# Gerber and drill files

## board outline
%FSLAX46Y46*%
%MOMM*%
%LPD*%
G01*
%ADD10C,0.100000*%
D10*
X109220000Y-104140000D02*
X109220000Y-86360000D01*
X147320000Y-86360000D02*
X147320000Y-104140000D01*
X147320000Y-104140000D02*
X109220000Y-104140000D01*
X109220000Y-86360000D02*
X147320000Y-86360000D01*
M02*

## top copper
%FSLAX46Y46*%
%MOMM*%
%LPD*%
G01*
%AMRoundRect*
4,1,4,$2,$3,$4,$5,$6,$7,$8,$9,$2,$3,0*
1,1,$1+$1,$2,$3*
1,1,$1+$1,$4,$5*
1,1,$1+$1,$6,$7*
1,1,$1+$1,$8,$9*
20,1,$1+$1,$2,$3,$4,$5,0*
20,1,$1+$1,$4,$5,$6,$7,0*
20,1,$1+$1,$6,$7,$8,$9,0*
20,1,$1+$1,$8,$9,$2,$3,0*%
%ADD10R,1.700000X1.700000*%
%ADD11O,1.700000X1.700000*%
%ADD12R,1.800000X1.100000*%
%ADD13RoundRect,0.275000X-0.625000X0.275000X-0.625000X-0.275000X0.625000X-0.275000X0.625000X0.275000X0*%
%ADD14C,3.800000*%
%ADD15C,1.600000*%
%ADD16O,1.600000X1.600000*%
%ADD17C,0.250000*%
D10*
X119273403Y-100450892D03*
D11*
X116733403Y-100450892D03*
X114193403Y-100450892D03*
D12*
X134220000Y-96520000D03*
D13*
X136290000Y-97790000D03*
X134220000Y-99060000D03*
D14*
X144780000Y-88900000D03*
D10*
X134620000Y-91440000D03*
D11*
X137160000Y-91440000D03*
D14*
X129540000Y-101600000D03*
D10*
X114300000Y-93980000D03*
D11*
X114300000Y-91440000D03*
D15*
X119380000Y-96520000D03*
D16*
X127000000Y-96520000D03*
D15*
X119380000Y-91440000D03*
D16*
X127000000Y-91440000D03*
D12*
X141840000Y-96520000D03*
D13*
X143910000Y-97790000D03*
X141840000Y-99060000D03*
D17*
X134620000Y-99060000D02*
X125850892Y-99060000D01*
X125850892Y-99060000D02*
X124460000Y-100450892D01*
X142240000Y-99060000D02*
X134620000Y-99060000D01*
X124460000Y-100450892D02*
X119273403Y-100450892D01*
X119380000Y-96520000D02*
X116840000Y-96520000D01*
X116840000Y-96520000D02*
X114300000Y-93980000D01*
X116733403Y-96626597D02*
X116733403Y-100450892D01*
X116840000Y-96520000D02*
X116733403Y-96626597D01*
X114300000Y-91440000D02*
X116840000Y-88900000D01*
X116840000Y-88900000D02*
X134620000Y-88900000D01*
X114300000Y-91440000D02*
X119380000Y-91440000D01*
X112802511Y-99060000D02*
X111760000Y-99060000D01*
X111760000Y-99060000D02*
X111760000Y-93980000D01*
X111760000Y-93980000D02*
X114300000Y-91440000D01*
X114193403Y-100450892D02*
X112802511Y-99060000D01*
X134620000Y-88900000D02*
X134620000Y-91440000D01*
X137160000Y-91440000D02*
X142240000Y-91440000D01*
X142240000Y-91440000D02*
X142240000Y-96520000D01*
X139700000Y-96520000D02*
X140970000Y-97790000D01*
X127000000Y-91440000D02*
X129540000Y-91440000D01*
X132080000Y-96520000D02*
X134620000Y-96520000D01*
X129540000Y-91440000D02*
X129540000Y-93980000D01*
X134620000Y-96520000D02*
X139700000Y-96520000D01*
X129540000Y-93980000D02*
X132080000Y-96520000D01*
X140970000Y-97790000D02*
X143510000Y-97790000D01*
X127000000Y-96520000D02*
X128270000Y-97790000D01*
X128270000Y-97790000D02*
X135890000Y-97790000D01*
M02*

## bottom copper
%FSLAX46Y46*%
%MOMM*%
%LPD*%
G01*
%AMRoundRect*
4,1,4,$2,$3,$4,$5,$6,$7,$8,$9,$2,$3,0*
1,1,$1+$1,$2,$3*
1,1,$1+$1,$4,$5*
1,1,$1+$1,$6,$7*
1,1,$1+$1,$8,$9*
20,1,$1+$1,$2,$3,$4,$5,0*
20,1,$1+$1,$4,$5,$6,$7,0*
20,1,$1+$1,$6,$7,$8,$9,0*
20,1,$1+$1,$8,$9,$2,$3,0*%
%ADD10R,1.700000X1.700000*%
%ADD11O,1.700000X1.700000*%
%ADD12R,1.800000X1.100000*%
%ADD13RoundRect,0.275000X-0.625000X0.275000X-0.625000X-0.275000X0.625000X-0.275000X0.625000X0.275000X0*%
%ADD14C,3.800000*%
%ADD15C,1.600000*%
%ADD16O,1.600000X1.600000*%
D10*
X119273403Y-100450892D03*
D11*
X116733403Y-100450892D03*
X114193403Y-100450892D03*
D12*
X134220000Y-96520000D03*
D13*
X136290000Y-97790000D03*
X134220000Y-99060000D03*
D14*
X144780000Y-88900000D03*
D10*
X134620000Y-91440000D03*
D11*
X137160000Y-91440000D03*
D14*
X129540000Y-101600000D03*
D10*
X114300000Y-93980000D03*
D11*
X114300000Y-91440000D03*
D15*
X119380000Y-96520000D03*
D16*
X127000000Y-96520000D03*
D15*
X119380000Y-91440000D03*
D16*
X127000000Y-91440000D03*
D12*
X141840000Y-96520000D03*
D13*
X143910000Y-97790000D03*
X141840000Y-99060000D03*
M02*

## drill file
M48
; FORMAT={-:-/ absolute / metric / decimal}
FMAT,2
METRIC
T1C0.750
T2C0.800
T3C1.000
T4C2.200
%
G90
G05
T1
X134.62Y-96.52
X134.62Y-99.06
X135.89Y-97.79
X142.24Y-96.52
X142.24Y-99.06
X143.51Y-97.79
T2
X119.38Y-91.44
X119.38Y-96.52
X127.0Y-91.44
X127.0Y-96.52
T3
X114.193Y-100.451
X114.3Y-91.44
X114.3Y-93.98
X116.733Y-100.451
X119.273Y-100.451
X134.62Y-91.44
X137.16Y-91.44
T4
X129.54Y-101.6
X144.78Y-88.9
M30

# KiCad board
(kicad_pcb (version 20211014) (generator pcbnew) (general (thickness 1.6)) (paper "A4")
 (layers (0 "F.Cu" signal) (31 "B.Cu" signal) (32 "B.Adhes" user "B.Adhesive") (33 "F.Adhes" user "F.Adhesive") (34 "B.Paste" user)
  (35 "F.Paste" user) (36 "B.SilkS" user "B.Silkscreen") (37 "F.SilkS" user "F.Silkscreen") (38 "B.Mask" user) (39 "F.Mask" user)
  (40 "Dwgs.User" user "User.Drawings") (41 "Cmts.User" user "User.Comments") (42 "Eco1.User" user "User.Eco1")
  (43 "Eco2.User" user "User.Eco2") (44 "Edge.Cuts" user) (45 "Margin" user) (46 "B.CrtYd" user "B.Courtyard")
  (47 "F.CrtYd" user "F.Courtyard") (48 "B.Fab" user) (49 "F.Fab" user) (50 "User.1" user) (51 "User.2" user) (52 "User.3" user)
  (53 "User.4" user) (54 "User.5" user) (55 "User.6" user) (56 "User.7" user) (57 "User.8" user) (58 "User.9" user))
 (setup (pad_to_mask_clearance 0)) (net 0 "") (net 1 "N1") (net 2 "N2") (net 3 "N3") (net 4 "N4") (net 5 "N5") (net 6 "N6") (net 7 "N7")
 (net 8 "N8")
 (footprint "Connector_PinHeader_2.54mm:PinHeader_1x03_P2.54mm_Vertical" (layer "F.Cu") (at 119.273403 100.450892 -90)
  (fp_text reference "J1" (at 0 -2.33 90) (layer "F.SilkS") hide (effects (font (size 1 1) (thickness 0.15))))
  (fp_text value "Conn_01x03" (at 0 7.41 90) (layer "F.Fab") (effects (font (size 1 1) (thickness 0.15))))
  (pad "1" thru_hole rect (at 0 0 270) (size 1.7 1.7) (drill 1) (layers *.Cu *.Mask) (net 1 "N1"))
  (pad "2" thru_hole oval (at 0 2.54 270) (size 1.7 1.7) (drill 1) (layers *.Cu *.Mask) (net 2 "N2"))
  (pad "3" thru_hole oval (at 0 5.08 270) (size 1.7 1.7) (drill 1) (layers *.Cu *.Mask) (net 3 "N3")))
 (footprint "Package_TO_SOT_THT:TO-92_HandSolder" (layer "F.Cu") (at 134.62 96.52 -90)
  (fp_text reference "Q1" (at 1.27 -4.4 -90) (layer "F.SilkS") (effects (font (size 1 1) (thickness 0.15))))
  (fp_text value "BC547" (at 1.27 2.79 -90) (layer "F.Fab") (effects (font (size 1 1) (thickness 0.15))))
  (pad "1" thru_hole rect (at 0 0 270) (size 1.1 1.8) (drill 0.75 (offset 0 0.4)) (layers *.Cu *.Mask) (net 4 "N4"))
  (pad "2" thru_hole roundrect (at 1.27 -1.27 270) (size 1.1 1.8) (drill 0.75 (offset 0 -0.4)) (layers *.Cu *.Mask) (roundrect_rratio 0.25)
   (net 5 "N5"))
  (pad "3" thru_hole roundrect (at 2.54 0 270) (size 1.1 1.8) (drill 0.75 (offset 0 0.4)) (layers *.Cu *.Mask) (roundrect_rratio 0.25)
   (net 1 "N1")))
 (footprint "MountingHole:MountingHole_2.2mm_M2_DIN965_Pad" (layer "F.Cu") (at 144.78 88.9)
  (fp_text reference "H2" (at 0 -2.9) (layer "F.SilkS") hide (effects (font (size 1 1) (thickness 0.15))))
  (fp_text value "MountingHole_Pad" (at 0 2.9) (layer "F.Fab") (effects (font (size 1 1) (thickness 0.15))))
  (pad "1" thru_hole circle (at 0 0) (size 3.8 3.8) (drill 2.2) (layers *.Cu *.Mask) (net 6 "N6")))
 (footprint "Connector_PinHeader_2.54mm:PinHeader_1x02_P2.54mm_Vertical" (layer "F.Cu") (at 134.62 91.44 90)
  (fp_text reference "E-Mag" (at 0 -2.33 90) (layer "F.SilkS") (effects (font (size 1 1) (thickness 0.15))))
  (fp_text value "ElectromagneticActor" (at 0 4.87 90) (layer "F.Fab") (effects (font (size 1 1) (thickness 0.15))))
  (pad "1" thru_hole rect (at 0 0 90) (size 1.7 1.7) (drill 1) (layers *.Cu *.Mask) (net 3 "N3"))
  (pad "2" thru_hole oval (at 0 2.54 90) (size 1.7 1.7) (drill 1) (layers *.Cu *.Mask) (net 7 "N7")))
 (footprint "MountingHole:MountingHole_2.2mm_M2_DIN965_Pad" (layer "F.Cu") (at 129.54 101.6)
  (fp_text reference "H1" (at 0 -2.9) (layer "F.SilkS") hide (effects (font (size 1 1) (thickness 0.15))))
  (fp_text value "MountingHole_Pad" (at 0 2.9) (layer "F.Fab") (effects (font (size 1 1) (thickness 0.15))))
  (pad "1" thru_hole circle (at 0 0) (size 3.8 3.8) (drill 2.2) (layers *.Cu *.Mask) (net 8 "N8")))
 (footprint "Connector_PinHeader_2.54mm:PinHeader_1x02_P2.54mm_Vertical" (layer "F.Cu") (at 114.3 93.98 180)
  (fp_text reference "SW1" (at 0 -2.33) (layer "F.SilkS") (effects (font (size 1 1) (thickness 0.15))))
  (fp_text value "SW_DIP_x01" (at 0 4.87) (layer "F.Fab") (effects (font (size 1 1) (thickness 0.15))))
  (pad "1" thru_hole rect (at 0 0 180) (size 1.7 1.7) (drill 1) (layers *.Cu *.Mask) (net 2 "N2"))
  (pad "2" thru_hole oval (at 0 2.54 180) (size 1.7 1.7) (drill 1) (layers *.Cu *.Mask) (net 3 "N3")))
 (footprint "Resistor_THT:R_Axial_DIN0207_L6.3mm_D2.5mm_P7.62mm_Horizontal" (layer "F.Cu") (at 119.38 96.52)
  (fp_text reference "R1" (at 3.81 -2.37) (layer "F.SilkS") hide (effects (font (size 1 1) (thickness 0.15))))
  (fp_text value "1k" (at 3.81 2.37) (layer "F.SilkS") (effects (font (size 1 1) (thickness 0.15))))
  (pad "1" thru_hole circle (at 0 0) (size 1.6 1.6) (drill 0.8) (layers *.Cu *.Mask) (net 2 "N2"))
  (pad "2" thru_hole oval (at 7.62 0) (size 1.6 1.6) (drill 0.8) (layers *.Cu *.Mask) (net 5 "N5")))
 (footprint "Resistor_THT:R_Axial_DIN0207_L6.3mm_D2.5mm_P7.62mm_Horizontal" (layer "F.Cu") (at 119.38 91.44)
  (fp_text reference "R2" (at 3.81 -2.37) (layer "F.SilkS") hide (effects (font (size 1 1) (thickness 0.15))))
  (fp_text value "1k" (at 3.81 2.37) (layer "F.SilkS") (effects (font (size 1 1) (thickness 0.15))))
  (pad "1" thru_hole circle (at 0 0) (size 1.6 1.6) (drill 0.8) (layers *.Cu *.Mask) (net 3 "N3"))
  (pad "2" thru_hole oval (at 7.62 0) (size 1.6 1.6) (drill 0.8) (layers *.Cu *.Mask) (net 4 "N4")))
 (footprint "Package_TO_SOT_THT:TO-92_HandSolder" (layer "F.Cu") (at 142.24 96.52 -90)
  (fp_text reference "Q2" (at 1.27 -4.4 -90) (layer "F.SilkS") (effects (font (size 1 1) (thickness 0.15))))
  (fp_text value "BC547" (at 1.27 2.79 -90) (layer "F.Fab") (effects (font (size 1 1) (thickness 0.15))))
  (pad "1" thru_hole rect (at 0 0 270) (size 1.1 1.8) (drill 0.75 (offset 0 0.4)) (layers *.Cu *.Mask) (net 7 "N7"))
  (pad "2" thru_hole roundrect (at 1.27 -1.27 270) (size 1.1 1.8) (drill 0.75 (offset 0 -0.4)) (layers *.Cu *.Mask) (roundrect_rratio 0.25)
   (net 4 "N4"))
  (pad "3" thru_hole roundrect (at 2.54 0 270) (size 1.1 1.8) (drill 0.75 (offset 0 0.4)) (layers *.Cu *.Mask) (roundrect_rratio 0.25)
   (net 1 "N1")))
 (gr_line (start 109.22 104.14) (end 109.22 86.36) (layer "Edge.Cuts") (width 0.1))
 (gr_line (start 147.32 86.36) (end 147.32 104.14) (layer "Edge.Cuts") (width 0.1))
 (gr_line (start 147.32 104.14) (end 109.22 104.14) (layer "Edge.Cuts") (width 0.1))
 (gr_line (start 109.22 86.36) (end 147.32 86.36) (layer "Edge.Cuts") (width 0.1))
 (segment (start 134.62 99.06) (end 125.850892 99.06) (width 0.25) (layer "F.Cu") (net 1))
 (segment (start 125.850892 99.06) (end 124.46 100.450892) (width 0.25) (layer "F.Cu") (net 1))
 (segment (start 142.24 99.06) (end 134.62 99.06) (width 0.25) (layer "F.Cu") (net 1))
 (segment (start 124.46 100.450892) (end 119.273403 100.450892) (width 0.25) (layer "F.Cu") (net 1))
 (segment (start 119.38 96.52) (end 116.84 96.52) (width 0.25) (layer "F.Cu") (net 2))
 (segment (start 116.84 96.52) (end 114.3 93.98) (width 0.25) (layer "F.Cu") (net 2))
 (segment (start 116.733403 96.626597) (end 116.733403 100.450892) (width 0.25) (layer "F.Cu") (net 2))
 (segment (start 116.84 96.52) (end 116.733403 96.626597) (width 0.25) (layer "F.Cu") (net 2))
 (segment (start 114.3 91.44) (end 116.84 88.9) (width 0.25) (layer "F.Cu") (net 3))
 (segment (start 116.84 88.9) (end 134.62 88.9) (width 0.25) (layer "F.Cu") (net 3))
 (segment (start 114.3 91.44) (end 119.38 91.44) (width 0.25) (layer "F.Cu") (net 3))
 (segment (start 112.802511 99.06) (end 111.76 99.06) (width 0.25) (layer "F.Cu") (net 3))
 (segment (start 111.76 99.06) (end 111.76 93.98) (width 0.25) (layer "F.Cu") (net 3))
 (segment (start 111.76 93.98) (end 114.3 91.44) (width 0.25) (layer "F.Cu") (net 3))
 (segment (start 114.193403 100.450892) (end 112.802511 99.06) (width 0.25) (layer "F.Cu") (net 3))
 (segment (start 134.62 88.9) (end 134.62 91.44) (width 0.25) (layer "F.Cu") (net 3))
 (segment (start 137.16 91.44) (end 142.24 91.44) (width 0.25) (layer "F.Cu") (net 7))
 (segment (start 142.24 91.44) (end 142.24 96.52) (width 0.25) (layer "F.Cu") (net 7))
 (segment (start 139.7 96.52) (end 140.97 97.79) (width 0.25) (layer "F.Cu") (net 4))
 (segment (start 127 91.44) (end 129.54 91.44) (width 0.25) (layer "F.Cu") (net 4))
 (segment (start 132.08 96.52) (end 134.62 96.52) (width 0.25) (layer "F.Cu") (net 4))
 (segment (start 129.54 91.44) (end 129.54 93.98) (width 0.25) (layer "F.Cu") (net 4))
 (segment (start 134.62 96.52) (end 139.7 96.52) (width 0.25) (layer "F.Cu") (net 4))
 (segment (start 129.54 93.98) (end 132.08 96.52) (width 0.25) (layer "F.Cu") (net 4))
 (segment (start 140.97 97.79) (end 143.51 97.79) (width 0.25) (layer "F.Cu") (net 4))
 (segment (start 127 96.52) (end 128.27 97.79) (width 0.25) (layer "F.Cu") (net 5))
 (segment (start 128.27 97.79) (end 135.89 97.79) (width 0.25) (layer "F.Cu") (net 5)))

